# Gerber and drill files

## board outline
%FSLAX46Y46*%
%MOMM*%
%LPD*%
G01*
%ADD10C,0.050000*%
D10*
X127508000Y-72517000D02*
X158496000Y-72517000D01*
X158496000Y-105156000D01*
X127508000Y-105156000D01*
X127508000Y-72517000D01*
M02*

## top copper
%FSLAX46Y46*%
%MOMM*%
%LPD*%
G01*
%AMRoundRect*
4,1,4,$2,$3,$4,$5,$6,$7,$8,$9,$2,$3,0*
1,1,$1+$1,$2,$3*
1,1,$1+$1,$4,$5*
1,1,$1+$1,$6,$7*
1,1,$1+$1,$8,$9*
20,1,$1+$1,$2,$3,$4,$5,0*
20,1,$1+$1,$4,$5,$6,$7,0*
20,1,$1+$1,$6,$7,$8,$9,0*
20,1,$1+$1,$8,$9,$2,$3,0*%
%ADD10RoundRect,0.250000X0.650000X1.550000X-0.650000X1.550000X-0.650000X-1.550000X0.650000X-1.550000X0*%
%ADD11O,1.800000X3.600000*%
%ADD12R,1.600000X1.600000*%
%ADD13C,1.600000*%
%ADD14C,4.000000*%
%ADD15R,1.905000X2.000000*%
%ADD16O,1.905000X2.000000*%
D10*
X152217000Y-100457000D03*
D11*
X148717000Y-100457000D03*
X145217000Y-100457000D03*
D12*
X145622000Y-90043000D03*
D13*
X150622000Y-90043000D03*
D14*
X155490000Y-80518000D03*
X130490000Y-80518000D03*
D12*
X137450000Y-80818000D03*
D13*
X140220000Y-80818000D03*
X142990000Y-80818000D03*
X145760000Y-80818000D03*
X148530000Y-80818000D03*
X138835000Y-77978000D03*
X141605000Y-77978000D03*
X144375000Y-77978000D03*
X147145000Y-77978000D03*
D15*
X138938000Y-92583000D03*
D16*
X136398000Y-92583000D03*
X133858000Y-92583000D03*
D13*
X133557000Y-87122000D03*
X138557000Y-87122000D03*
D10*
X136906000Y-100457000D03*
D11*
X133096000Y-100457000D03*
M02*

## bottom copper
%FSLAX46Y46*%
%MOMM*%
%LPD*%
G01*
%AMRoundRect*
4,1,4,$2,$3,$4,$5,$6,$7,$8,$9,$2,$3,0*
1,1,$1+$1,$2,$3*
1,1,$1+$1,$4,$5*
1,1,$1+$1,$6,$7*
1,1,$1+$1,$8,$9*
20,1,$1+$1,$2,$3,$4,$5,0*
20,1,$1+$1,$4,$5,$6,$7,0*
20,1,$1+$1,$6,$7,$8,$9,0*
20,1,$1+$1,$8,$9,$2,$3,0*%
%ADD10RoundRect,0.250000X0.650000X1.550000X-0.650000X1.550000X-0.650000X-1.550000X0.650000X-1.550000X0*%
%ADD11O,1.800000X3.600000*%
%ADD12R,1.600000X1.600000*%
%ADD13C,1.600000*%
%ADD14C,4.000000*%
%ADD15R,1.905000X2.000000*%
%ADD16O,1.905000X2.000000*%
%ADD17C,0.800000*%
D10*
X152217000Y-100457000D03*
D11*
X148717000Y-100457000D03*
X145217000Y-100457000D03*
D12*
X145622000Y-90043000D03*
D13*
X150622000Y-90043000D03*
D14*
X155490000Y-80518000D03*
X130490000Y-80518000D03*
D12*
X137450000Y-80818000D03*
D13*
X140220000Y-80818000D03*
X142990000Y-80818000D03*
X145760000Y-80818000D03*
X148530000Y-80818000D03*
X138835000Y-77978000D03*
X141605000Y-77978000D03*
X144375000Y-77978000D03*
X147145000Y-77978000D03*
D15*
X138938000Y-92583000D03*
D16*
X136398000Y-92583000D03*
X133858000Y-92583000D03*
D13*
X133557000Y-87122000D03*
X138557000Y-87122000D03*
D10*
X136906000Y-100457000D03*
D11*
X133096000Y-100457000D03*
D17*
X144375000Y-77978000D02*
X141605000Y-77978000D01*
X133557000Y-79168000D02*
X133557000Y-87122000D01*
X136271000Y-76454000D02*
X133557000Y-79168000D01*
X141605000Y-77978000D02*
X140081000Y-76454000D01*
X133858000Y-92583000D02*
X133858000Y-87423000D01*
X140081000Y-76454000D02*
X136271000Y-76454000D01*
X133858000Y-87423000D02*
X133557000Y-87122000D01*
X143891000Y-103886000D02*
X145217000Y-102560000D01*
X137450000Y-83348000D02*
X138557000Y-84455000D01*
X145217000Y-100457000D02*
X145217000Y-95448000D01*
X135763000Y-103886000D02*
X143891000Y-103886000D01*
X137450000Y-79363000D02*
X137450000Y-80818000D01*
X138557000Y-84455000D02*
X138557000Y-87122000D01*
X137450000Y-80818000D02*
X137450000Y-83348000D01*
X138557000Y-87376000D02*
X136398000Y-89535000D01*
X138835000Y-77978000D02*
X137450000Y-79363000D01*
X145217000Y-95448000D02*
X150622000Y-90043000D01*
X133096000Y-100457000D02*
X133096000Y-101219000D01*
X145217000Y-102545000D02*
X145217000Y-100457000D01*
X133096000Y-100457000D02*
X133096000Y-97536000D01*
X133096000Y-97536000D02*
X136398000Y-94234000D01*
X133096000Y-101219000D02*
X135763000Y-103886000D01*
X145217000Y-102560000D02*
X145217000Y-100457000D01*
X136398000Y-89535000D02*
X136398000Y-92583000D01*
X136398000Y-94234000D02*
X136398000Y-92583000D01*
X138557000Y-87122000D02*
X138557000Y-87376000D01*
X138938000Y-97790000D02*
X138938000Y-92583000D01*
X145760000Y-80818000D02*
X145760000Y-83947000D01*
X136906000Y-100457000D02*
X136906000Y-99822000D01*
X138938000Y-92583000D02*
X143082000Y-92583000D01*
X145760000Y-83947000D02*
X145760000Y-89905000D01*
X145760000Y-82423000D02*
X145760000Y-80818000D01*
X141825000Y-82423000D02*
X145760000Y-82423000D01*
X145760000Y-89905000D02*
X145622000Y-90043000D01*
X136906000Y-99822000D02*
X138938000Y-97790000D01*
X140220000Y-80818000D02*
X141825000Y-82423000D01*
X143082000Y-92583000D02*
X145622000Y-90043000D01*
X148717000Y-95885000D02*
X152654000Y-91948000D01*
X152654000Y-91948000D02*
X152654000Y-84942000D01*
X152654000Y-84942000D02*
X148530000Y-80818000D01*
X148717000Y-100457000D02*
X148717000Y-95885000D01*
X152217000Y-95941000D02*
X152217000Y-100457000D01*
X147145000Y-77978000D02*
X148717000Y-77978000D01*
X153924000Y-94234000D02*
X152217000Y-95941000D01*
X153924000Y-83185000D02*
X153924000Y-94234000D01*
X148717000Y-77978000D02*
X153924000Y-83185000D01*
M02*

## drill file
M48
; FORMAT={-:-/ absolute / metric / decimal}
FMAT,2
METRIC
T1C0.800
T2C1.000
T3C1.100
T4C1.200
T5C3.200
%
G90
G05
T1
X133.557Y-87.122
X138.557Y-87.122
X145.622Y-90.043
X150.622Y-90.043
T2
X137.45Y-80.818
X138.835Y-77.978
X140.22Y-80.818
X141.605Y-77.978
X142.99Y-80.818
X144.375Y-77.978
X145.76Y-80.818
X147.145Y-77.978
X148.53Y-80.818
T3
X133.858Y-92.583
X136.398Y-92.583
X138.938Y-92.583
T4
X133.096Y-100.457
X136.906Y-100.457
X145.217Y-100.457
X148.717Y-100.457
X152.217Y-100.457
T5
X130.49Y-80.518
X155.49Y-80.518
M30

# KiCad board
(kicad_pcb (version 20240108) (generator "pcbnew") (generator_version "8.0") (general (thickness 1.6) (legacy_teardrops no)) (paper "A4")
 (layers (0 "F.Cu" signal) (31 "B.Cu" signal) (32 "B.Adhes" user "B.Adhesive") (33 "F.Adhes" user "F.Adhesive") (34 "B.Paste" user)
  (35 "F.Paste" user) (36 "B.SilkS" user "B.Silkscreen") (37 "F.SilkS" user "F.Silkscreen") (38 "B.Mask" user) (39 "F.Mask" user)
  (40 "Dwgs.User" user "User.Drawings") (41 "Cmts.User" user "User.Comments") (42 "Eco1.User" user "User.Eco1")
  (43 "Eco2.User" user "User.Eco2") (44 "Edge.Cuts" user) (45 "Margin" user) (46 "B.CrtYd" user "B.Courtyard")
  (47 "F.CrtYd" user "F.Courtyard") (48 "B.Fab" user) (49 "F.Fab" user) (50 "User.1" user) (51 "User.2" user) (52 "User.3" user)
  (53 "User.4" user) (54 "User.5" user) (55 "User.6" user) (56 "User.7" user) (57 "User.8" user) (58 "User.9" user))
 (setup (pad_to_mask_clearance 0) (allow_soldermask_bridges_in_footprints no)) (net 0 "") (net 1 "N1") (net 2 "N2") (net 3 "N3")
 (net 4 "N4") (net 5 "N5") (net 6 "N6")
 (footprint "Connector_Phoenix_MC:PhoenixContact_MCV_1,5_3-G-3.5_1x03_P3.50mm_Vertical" (layer "F.Cu") (at 152.217 100.457 180)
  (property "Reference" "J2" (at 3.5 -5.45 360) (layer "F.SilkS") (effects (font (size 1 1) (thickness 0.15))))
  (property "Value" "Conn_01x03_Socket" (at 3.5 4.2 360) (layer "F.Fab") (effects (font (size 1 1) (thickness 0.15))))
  (pad "1" thru_hole roundrect (at 0 0 180) (size 1.8 3.6) (drill 1.2) (layers "*.Cu" "*.Mask") (remove_unused_layers no)
   (roundrect_rratio 0.138889) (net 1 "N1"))
  (pad "2" thru_hole oval (at 3.5 0 180) (size 1.8 3.6) (drill 1.2) (layers "*.Cu" "*.Mask") (remove_unused_layers no) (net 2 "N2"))
  (pad "3" thru_hole oval (at 7 0 180) (size 1.8 3.6) (drill 1.2) (layers "*.Cu" "*.Mask") (remove_unused_layers no) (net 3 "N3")))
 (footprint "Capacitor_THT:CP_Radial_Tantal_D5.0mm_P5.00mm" (layer "F.Cu") (at 145.622 90.043)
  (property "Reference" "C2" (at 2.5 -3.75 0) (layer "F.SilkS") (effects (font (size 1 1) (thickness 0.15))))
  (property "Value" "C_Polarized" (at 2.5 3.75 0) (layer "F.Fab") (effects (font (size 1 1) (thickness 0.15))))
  (pad "1" thru_hole rect (at 0 0) (size 1.6 1.6) (drill 0.8) (layers "*.Cu" "*.Mask") (remove_unused_layers no) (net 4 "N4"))
  (pad "2" thru_hole circle (at 5 0) (size 1.6 1.6) (drill 0.8) (layers "*.Cu" "*.Mask") (remove_unused_layers no) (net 3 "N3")))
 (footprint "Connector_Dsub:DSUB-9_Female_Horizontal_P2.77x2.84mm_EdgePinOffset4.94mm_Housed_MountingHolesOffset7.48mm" (layer "F.Cu")
  (at 137.45 80.818 180)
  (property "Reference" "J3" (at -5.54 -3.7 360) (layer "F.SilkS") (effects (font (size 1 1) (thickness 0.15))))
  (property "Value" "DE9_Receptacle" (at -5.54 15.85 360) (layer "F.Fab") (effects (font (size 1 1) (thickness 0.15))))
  (pad "0" thru_hole circle (at -18.04 0.3 180) (size 4 4) (drill 3.2) (layers "*.Cu" "*.Mask") (remove_unused_layers no))
  (pad "0" thru_hole circle (at 6.96 0.3 180) (size 4 4) (drill 3.2) (layers "*.Cu" "*.Mask") (remove_unused_layers no))
  (pad "1" thru_hole rect (at 0 0 180) (size 1.6 1.6) (drill 1) (layers "*.Cu" "*.Mask") (remove_unused_layers no) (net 3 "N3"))
  (pad "2" thru_hole circle (at -2.77 0 180) (size 1.6 1.6) (drill 1) (layers "*.Cu" "*.Mask") (remove_unused_layers no) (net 4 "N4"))
  (pad "3" thru_hole circle (at -5.54 0 180) (size 1.6 1.6) (drill 1) (layers "*.Cu" "*.Mask") (remove_unused_layers no) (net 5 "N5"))
  (pad "4" thru_hole circle (at -8.31 0 180) (size 1.6 1.6) (drill 1) (layers "*.Cu" "*.Mask") (remove_unused_layers no) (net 4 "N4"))
  (pad "5" thru_hole circle (at -11.08 0 180) (size 1.6 1.6) (drill 1) (layers "*.Cu" "*.Mask") (remove_unused_layers no) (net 2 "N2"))
  (pad "6" thru_hole circle (at -1.385 2.84 180) (size 1.6 1.6) (drill 1) (layers "*.Cu" "*.Mask") (remove_unused_layers no) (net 3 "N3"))
  (pad "7" thru_hole circle (at -4.155 2.84 180) (size 1.6 1.6) (drill 1) (layers "*.Cu" "*.Mask") (remove_unused_layers no) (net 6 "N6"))
  (pad "8" thru_hole circle (at -6.925 2.84 180) (size 1.6 1.6) (drill 1) (layers "*.Cu" "*.Mask") (remove_unused_layers no) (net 6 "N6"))
  (pad "9" thru_hole circle (at -9.695 2.84 180) (size 1.6 1.6) (drill 1) (layers "*.Cu" "*.Mask") (remove_unused_layers no) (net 1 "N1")))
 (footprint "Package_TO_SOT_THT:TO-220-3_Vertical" (layer "F.Cu") (at 138.938 92.583 180)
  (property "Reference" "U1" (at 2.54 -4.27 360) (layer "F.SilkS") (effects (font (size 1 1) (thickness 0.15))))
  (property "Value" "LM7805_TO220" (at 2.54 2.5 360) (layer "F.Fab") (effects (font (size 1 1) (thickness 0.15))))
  (pad "1" thru_hole rect (at 0 0 180) (size 1.905 2) (drill 1.1) (layers "*.Cu" "*.Mask") (remove_unused_layers no) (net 4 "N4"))
  (pad "2" thru_hole oval (at 2.54 0 180) (size 1.905 2) (drill 1.1) (layers "*.Cu" "*.Mask") (remove_unused_layers no) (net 3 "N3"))
  (pad "3" thru_hole oval (at 5.08 0 180) (size 1.905 2) (drill 1.1) (layers "*.Cu" "*.Mask") (remove_unused_layers no) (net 6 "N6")))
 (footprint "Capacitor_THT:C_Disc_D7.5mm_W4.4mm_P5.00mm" (layer "F.Cu") (at 133.557 87.122)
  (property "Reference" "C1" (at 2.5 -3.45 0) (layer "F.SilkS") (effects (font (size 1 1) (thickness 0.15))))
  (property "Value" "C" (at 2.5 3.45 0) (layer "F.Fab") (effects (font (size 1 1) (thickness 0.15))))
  (pad "1" thru_hole circle (at 0 0) (size 1.6 1.6) (drill 0.8) (layers "*.Cu" "*.Mask") (remove_unused_layers no) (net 6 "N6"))
  (pad "2" thru_hole circle (at 5 0) (size 1.6 1.6) (drill 0.8) (layers "*.Cu" "*.Mask") (remove_unused_layers no) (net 3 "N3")))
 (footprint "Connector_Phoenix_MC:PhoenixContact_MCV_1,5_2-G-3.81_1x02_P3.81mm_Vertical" (layer "F.Cu") (at 136.906 100.457 180)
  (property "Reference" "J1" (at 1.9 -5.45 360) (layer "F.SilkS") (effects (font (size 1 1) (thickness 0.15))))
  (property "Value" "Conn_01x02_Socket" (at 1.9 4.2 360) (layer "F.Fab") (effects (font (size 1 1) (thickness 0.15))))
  (pad "1" thru_hole roundrect (at 0 0 180) (size 1.8 3.6) (drill 1.2) (layers "*.Cu" "*.Mask") (remove_unused_layers no)
   (roundrect_rratio 0.138889) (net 4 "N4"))
  (pad "2" thru_hole oval (at 3.81 0 180) (size 1.8 3.6) (drill 1.2) (layers "*.Cu" "*.Mask") (remove_unused_layers no) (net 3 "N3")))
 (gr_rect (start 127.508 72.517) (end 158.496 105.156) (stroke (width 0.05) (type default)) (fill none) (layer "Edge.Cuts"))
 (segment (start 144.375 77.978) (end 141.605 77.978) (width 0.8) (layer "B.Cu") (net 6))
 (segment (start 133.557 79.168) (end 133.557 87.122) (width 0.8) (layer "B.Cu") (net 6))
 (segment (start 136.271 76.454) (end 133.557 79.168) (width 0.8) (layer "B.Cu") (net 6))
 (segment (start 141.605 77.978) (end 140.081 76.454) (width 0.8) (layer "B.Cu") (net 6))
 (segment (start 133.858 92.583) (end 133.858 87.423) (width 0.8) (layer "B.Cu") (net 6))
 (segment (start 140.081 76.454) (end 136.271 76.454) (width 0.8) (layer "B.Cu") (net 6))
 (segment (start 133.858 87.423) (end 133.557 87.122) (width 0.8) (layer "B.Cu") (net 6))
 (segment (start 143.891 103.886) (end 145.217 102.56) (width 0.8) (layer "B.Cu") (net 3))
 (segment (start 137.45 83.348) (end 138.557 84.455) (width 0.8) (layer "B.Cu") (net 3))
 (segment (start 145.217 100.457) (end 145.217 95.448) (width 0.8) (layer "B.Cu") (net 3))
 (segment (start 135.763 103.886) (end 143.891 103.886) (width 0.8) (layer "B.Cu") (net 3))
 (segment (start 137.45 79.363) (end 137.45 80.818) (width 0.8) (layer "B.Cu") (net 3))
 (segment (start 138.557 84.455) (end 138.557 87.122) (width 0.8) (layer "B.Cu") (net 3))
 (segment (start 137.45 80.818) (end 137.45 83.348) (width 0.8) (layer "B.Cu") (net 3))
 (segment (start 138.557 87.376) (end 136.398 89.535) (width 0.8) (layer "B.Cu") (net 3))
 (segment (start 138.835 77.978) (end 137.45 79.363) (width 0.8) (layer "B.Cu") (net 3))
 (segment (start 145.217 95.448) (end 150.622 90.043) (width 0.8) (layer "B.Cu") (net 3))
 (segment (start 133.096 100.457) (end 133.096 101.219) (width 0.8) (layer "B.Cu") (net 3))
 (segment (start 145.217 102.545) (end 145.217 100.457) (width 0.8) (layer "B.Cu") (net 3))
 (segment (start 133.096 100.457) (end 133.096 97.536) (width 0.8) (layer "B.Cu") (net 3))
 (segment (start 133.096 97.536) (end 136.398 94.234) (width 0.8) (layer "B.Cu") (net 3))
 (segment (start 133.096 101.219) (end 135.763 103.886) (width 0.8) (layer "B.Cu") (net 3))
 (segment (start 145.217 102.56) (end 145.217 100.457) (width 0.8) (layer "B.Cu") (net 3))
 (segment (start 136.398 89.535) (end 136.398 92.583) (width 0.8) (layer "B.Cu") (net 3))
 (segment (start 136.398 94.234) (end 136.398 92.583) (width 0.8) (layer "B.Cu") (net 3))
 (segment (start 138.557 87.122) (end 138.557 87.376) (width 0.8) (layer "B.Cu") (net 3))
 (segment (start 138.938 97.79) (end 138.938 92.583) (width 0.8) (layer "B.Cu") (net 4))
 (segment (start 145.76 80.818) (end 145.76 83.947) (width 0.8) (layer "B.Cu") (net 4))
 (segment (start 136.906 100.457) (end 136.906 99.822) (width 0.8) (layer "B.Cu") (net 4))
 (segment (start 138.938 92.583) (end 143.082 92.583) (width 0.8) (layer "B.Cu") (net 4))
 (segment (start 145.76 83.947) (end 145.76 89.905) (width 0.8) (layer "B.Cu") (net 4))
 (segment (start 145.76 82.423) (end 145.76 80.818) (width 0.8) (layer "B.Cu") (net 4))
 (segment (start 141.825 82.423) (end 145.76 82.423) (width 0.8) (layer "B.Cu") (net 4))
 (segment (start 145.76 89.905) (end 145.622 90.043) (width 0.8) (layer "B.Cu") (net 4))
 (segment (start 136.906 99.822) (end 138.938 97.79) (width 0.8) (layer "B.Cu") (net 4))
 (segment (start 140.22 80.818) (end 141.825 82.423) (width 0.8) (layer "B.Cu") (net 4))
 (segment (start 143.082 92.583) (end 145.622 90.043) (width 0.8) (layer "B.Cu") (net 4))
 (segment (start 148.717 95.885) (end 152.654 91.948) (width 0.8) (layer "B.Cu") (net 2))
 (segment (start 152.654 91.948) (end 152.654 84.942) (width 0.8) (layer "B.Cu") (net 2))
 (segment (start 152.654 84.942) (end 148.53 80.818) (width 0.8) (layer "B.Cu") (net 2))
 (segment (start 148.717 100.457) (end 148.717 95.885) (width 0.8) (layer "B.Cu") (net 2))
 (segment (start 152.217 95.941) (end 152.217 100.457) (width 0.8) (layer "B.Cu") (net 1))
 (segment (start 147.145 77.978) (end 148.717 77.978) (width 0.8) (layer "B.Cu") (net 1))
 (segment (start 153.924 94.234) (end 152.217 95.941) (width 0.8) (layer "B.Cu") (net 1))
 (segment (start 153.924 83.185) (end 153.924 94.234) (width 0.8) (layer "B.Cu") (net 1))
 (segment (start 148.717 77.978) (end 153.924 83.185) (width 0.8) (layer "B.Cu") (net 1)))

